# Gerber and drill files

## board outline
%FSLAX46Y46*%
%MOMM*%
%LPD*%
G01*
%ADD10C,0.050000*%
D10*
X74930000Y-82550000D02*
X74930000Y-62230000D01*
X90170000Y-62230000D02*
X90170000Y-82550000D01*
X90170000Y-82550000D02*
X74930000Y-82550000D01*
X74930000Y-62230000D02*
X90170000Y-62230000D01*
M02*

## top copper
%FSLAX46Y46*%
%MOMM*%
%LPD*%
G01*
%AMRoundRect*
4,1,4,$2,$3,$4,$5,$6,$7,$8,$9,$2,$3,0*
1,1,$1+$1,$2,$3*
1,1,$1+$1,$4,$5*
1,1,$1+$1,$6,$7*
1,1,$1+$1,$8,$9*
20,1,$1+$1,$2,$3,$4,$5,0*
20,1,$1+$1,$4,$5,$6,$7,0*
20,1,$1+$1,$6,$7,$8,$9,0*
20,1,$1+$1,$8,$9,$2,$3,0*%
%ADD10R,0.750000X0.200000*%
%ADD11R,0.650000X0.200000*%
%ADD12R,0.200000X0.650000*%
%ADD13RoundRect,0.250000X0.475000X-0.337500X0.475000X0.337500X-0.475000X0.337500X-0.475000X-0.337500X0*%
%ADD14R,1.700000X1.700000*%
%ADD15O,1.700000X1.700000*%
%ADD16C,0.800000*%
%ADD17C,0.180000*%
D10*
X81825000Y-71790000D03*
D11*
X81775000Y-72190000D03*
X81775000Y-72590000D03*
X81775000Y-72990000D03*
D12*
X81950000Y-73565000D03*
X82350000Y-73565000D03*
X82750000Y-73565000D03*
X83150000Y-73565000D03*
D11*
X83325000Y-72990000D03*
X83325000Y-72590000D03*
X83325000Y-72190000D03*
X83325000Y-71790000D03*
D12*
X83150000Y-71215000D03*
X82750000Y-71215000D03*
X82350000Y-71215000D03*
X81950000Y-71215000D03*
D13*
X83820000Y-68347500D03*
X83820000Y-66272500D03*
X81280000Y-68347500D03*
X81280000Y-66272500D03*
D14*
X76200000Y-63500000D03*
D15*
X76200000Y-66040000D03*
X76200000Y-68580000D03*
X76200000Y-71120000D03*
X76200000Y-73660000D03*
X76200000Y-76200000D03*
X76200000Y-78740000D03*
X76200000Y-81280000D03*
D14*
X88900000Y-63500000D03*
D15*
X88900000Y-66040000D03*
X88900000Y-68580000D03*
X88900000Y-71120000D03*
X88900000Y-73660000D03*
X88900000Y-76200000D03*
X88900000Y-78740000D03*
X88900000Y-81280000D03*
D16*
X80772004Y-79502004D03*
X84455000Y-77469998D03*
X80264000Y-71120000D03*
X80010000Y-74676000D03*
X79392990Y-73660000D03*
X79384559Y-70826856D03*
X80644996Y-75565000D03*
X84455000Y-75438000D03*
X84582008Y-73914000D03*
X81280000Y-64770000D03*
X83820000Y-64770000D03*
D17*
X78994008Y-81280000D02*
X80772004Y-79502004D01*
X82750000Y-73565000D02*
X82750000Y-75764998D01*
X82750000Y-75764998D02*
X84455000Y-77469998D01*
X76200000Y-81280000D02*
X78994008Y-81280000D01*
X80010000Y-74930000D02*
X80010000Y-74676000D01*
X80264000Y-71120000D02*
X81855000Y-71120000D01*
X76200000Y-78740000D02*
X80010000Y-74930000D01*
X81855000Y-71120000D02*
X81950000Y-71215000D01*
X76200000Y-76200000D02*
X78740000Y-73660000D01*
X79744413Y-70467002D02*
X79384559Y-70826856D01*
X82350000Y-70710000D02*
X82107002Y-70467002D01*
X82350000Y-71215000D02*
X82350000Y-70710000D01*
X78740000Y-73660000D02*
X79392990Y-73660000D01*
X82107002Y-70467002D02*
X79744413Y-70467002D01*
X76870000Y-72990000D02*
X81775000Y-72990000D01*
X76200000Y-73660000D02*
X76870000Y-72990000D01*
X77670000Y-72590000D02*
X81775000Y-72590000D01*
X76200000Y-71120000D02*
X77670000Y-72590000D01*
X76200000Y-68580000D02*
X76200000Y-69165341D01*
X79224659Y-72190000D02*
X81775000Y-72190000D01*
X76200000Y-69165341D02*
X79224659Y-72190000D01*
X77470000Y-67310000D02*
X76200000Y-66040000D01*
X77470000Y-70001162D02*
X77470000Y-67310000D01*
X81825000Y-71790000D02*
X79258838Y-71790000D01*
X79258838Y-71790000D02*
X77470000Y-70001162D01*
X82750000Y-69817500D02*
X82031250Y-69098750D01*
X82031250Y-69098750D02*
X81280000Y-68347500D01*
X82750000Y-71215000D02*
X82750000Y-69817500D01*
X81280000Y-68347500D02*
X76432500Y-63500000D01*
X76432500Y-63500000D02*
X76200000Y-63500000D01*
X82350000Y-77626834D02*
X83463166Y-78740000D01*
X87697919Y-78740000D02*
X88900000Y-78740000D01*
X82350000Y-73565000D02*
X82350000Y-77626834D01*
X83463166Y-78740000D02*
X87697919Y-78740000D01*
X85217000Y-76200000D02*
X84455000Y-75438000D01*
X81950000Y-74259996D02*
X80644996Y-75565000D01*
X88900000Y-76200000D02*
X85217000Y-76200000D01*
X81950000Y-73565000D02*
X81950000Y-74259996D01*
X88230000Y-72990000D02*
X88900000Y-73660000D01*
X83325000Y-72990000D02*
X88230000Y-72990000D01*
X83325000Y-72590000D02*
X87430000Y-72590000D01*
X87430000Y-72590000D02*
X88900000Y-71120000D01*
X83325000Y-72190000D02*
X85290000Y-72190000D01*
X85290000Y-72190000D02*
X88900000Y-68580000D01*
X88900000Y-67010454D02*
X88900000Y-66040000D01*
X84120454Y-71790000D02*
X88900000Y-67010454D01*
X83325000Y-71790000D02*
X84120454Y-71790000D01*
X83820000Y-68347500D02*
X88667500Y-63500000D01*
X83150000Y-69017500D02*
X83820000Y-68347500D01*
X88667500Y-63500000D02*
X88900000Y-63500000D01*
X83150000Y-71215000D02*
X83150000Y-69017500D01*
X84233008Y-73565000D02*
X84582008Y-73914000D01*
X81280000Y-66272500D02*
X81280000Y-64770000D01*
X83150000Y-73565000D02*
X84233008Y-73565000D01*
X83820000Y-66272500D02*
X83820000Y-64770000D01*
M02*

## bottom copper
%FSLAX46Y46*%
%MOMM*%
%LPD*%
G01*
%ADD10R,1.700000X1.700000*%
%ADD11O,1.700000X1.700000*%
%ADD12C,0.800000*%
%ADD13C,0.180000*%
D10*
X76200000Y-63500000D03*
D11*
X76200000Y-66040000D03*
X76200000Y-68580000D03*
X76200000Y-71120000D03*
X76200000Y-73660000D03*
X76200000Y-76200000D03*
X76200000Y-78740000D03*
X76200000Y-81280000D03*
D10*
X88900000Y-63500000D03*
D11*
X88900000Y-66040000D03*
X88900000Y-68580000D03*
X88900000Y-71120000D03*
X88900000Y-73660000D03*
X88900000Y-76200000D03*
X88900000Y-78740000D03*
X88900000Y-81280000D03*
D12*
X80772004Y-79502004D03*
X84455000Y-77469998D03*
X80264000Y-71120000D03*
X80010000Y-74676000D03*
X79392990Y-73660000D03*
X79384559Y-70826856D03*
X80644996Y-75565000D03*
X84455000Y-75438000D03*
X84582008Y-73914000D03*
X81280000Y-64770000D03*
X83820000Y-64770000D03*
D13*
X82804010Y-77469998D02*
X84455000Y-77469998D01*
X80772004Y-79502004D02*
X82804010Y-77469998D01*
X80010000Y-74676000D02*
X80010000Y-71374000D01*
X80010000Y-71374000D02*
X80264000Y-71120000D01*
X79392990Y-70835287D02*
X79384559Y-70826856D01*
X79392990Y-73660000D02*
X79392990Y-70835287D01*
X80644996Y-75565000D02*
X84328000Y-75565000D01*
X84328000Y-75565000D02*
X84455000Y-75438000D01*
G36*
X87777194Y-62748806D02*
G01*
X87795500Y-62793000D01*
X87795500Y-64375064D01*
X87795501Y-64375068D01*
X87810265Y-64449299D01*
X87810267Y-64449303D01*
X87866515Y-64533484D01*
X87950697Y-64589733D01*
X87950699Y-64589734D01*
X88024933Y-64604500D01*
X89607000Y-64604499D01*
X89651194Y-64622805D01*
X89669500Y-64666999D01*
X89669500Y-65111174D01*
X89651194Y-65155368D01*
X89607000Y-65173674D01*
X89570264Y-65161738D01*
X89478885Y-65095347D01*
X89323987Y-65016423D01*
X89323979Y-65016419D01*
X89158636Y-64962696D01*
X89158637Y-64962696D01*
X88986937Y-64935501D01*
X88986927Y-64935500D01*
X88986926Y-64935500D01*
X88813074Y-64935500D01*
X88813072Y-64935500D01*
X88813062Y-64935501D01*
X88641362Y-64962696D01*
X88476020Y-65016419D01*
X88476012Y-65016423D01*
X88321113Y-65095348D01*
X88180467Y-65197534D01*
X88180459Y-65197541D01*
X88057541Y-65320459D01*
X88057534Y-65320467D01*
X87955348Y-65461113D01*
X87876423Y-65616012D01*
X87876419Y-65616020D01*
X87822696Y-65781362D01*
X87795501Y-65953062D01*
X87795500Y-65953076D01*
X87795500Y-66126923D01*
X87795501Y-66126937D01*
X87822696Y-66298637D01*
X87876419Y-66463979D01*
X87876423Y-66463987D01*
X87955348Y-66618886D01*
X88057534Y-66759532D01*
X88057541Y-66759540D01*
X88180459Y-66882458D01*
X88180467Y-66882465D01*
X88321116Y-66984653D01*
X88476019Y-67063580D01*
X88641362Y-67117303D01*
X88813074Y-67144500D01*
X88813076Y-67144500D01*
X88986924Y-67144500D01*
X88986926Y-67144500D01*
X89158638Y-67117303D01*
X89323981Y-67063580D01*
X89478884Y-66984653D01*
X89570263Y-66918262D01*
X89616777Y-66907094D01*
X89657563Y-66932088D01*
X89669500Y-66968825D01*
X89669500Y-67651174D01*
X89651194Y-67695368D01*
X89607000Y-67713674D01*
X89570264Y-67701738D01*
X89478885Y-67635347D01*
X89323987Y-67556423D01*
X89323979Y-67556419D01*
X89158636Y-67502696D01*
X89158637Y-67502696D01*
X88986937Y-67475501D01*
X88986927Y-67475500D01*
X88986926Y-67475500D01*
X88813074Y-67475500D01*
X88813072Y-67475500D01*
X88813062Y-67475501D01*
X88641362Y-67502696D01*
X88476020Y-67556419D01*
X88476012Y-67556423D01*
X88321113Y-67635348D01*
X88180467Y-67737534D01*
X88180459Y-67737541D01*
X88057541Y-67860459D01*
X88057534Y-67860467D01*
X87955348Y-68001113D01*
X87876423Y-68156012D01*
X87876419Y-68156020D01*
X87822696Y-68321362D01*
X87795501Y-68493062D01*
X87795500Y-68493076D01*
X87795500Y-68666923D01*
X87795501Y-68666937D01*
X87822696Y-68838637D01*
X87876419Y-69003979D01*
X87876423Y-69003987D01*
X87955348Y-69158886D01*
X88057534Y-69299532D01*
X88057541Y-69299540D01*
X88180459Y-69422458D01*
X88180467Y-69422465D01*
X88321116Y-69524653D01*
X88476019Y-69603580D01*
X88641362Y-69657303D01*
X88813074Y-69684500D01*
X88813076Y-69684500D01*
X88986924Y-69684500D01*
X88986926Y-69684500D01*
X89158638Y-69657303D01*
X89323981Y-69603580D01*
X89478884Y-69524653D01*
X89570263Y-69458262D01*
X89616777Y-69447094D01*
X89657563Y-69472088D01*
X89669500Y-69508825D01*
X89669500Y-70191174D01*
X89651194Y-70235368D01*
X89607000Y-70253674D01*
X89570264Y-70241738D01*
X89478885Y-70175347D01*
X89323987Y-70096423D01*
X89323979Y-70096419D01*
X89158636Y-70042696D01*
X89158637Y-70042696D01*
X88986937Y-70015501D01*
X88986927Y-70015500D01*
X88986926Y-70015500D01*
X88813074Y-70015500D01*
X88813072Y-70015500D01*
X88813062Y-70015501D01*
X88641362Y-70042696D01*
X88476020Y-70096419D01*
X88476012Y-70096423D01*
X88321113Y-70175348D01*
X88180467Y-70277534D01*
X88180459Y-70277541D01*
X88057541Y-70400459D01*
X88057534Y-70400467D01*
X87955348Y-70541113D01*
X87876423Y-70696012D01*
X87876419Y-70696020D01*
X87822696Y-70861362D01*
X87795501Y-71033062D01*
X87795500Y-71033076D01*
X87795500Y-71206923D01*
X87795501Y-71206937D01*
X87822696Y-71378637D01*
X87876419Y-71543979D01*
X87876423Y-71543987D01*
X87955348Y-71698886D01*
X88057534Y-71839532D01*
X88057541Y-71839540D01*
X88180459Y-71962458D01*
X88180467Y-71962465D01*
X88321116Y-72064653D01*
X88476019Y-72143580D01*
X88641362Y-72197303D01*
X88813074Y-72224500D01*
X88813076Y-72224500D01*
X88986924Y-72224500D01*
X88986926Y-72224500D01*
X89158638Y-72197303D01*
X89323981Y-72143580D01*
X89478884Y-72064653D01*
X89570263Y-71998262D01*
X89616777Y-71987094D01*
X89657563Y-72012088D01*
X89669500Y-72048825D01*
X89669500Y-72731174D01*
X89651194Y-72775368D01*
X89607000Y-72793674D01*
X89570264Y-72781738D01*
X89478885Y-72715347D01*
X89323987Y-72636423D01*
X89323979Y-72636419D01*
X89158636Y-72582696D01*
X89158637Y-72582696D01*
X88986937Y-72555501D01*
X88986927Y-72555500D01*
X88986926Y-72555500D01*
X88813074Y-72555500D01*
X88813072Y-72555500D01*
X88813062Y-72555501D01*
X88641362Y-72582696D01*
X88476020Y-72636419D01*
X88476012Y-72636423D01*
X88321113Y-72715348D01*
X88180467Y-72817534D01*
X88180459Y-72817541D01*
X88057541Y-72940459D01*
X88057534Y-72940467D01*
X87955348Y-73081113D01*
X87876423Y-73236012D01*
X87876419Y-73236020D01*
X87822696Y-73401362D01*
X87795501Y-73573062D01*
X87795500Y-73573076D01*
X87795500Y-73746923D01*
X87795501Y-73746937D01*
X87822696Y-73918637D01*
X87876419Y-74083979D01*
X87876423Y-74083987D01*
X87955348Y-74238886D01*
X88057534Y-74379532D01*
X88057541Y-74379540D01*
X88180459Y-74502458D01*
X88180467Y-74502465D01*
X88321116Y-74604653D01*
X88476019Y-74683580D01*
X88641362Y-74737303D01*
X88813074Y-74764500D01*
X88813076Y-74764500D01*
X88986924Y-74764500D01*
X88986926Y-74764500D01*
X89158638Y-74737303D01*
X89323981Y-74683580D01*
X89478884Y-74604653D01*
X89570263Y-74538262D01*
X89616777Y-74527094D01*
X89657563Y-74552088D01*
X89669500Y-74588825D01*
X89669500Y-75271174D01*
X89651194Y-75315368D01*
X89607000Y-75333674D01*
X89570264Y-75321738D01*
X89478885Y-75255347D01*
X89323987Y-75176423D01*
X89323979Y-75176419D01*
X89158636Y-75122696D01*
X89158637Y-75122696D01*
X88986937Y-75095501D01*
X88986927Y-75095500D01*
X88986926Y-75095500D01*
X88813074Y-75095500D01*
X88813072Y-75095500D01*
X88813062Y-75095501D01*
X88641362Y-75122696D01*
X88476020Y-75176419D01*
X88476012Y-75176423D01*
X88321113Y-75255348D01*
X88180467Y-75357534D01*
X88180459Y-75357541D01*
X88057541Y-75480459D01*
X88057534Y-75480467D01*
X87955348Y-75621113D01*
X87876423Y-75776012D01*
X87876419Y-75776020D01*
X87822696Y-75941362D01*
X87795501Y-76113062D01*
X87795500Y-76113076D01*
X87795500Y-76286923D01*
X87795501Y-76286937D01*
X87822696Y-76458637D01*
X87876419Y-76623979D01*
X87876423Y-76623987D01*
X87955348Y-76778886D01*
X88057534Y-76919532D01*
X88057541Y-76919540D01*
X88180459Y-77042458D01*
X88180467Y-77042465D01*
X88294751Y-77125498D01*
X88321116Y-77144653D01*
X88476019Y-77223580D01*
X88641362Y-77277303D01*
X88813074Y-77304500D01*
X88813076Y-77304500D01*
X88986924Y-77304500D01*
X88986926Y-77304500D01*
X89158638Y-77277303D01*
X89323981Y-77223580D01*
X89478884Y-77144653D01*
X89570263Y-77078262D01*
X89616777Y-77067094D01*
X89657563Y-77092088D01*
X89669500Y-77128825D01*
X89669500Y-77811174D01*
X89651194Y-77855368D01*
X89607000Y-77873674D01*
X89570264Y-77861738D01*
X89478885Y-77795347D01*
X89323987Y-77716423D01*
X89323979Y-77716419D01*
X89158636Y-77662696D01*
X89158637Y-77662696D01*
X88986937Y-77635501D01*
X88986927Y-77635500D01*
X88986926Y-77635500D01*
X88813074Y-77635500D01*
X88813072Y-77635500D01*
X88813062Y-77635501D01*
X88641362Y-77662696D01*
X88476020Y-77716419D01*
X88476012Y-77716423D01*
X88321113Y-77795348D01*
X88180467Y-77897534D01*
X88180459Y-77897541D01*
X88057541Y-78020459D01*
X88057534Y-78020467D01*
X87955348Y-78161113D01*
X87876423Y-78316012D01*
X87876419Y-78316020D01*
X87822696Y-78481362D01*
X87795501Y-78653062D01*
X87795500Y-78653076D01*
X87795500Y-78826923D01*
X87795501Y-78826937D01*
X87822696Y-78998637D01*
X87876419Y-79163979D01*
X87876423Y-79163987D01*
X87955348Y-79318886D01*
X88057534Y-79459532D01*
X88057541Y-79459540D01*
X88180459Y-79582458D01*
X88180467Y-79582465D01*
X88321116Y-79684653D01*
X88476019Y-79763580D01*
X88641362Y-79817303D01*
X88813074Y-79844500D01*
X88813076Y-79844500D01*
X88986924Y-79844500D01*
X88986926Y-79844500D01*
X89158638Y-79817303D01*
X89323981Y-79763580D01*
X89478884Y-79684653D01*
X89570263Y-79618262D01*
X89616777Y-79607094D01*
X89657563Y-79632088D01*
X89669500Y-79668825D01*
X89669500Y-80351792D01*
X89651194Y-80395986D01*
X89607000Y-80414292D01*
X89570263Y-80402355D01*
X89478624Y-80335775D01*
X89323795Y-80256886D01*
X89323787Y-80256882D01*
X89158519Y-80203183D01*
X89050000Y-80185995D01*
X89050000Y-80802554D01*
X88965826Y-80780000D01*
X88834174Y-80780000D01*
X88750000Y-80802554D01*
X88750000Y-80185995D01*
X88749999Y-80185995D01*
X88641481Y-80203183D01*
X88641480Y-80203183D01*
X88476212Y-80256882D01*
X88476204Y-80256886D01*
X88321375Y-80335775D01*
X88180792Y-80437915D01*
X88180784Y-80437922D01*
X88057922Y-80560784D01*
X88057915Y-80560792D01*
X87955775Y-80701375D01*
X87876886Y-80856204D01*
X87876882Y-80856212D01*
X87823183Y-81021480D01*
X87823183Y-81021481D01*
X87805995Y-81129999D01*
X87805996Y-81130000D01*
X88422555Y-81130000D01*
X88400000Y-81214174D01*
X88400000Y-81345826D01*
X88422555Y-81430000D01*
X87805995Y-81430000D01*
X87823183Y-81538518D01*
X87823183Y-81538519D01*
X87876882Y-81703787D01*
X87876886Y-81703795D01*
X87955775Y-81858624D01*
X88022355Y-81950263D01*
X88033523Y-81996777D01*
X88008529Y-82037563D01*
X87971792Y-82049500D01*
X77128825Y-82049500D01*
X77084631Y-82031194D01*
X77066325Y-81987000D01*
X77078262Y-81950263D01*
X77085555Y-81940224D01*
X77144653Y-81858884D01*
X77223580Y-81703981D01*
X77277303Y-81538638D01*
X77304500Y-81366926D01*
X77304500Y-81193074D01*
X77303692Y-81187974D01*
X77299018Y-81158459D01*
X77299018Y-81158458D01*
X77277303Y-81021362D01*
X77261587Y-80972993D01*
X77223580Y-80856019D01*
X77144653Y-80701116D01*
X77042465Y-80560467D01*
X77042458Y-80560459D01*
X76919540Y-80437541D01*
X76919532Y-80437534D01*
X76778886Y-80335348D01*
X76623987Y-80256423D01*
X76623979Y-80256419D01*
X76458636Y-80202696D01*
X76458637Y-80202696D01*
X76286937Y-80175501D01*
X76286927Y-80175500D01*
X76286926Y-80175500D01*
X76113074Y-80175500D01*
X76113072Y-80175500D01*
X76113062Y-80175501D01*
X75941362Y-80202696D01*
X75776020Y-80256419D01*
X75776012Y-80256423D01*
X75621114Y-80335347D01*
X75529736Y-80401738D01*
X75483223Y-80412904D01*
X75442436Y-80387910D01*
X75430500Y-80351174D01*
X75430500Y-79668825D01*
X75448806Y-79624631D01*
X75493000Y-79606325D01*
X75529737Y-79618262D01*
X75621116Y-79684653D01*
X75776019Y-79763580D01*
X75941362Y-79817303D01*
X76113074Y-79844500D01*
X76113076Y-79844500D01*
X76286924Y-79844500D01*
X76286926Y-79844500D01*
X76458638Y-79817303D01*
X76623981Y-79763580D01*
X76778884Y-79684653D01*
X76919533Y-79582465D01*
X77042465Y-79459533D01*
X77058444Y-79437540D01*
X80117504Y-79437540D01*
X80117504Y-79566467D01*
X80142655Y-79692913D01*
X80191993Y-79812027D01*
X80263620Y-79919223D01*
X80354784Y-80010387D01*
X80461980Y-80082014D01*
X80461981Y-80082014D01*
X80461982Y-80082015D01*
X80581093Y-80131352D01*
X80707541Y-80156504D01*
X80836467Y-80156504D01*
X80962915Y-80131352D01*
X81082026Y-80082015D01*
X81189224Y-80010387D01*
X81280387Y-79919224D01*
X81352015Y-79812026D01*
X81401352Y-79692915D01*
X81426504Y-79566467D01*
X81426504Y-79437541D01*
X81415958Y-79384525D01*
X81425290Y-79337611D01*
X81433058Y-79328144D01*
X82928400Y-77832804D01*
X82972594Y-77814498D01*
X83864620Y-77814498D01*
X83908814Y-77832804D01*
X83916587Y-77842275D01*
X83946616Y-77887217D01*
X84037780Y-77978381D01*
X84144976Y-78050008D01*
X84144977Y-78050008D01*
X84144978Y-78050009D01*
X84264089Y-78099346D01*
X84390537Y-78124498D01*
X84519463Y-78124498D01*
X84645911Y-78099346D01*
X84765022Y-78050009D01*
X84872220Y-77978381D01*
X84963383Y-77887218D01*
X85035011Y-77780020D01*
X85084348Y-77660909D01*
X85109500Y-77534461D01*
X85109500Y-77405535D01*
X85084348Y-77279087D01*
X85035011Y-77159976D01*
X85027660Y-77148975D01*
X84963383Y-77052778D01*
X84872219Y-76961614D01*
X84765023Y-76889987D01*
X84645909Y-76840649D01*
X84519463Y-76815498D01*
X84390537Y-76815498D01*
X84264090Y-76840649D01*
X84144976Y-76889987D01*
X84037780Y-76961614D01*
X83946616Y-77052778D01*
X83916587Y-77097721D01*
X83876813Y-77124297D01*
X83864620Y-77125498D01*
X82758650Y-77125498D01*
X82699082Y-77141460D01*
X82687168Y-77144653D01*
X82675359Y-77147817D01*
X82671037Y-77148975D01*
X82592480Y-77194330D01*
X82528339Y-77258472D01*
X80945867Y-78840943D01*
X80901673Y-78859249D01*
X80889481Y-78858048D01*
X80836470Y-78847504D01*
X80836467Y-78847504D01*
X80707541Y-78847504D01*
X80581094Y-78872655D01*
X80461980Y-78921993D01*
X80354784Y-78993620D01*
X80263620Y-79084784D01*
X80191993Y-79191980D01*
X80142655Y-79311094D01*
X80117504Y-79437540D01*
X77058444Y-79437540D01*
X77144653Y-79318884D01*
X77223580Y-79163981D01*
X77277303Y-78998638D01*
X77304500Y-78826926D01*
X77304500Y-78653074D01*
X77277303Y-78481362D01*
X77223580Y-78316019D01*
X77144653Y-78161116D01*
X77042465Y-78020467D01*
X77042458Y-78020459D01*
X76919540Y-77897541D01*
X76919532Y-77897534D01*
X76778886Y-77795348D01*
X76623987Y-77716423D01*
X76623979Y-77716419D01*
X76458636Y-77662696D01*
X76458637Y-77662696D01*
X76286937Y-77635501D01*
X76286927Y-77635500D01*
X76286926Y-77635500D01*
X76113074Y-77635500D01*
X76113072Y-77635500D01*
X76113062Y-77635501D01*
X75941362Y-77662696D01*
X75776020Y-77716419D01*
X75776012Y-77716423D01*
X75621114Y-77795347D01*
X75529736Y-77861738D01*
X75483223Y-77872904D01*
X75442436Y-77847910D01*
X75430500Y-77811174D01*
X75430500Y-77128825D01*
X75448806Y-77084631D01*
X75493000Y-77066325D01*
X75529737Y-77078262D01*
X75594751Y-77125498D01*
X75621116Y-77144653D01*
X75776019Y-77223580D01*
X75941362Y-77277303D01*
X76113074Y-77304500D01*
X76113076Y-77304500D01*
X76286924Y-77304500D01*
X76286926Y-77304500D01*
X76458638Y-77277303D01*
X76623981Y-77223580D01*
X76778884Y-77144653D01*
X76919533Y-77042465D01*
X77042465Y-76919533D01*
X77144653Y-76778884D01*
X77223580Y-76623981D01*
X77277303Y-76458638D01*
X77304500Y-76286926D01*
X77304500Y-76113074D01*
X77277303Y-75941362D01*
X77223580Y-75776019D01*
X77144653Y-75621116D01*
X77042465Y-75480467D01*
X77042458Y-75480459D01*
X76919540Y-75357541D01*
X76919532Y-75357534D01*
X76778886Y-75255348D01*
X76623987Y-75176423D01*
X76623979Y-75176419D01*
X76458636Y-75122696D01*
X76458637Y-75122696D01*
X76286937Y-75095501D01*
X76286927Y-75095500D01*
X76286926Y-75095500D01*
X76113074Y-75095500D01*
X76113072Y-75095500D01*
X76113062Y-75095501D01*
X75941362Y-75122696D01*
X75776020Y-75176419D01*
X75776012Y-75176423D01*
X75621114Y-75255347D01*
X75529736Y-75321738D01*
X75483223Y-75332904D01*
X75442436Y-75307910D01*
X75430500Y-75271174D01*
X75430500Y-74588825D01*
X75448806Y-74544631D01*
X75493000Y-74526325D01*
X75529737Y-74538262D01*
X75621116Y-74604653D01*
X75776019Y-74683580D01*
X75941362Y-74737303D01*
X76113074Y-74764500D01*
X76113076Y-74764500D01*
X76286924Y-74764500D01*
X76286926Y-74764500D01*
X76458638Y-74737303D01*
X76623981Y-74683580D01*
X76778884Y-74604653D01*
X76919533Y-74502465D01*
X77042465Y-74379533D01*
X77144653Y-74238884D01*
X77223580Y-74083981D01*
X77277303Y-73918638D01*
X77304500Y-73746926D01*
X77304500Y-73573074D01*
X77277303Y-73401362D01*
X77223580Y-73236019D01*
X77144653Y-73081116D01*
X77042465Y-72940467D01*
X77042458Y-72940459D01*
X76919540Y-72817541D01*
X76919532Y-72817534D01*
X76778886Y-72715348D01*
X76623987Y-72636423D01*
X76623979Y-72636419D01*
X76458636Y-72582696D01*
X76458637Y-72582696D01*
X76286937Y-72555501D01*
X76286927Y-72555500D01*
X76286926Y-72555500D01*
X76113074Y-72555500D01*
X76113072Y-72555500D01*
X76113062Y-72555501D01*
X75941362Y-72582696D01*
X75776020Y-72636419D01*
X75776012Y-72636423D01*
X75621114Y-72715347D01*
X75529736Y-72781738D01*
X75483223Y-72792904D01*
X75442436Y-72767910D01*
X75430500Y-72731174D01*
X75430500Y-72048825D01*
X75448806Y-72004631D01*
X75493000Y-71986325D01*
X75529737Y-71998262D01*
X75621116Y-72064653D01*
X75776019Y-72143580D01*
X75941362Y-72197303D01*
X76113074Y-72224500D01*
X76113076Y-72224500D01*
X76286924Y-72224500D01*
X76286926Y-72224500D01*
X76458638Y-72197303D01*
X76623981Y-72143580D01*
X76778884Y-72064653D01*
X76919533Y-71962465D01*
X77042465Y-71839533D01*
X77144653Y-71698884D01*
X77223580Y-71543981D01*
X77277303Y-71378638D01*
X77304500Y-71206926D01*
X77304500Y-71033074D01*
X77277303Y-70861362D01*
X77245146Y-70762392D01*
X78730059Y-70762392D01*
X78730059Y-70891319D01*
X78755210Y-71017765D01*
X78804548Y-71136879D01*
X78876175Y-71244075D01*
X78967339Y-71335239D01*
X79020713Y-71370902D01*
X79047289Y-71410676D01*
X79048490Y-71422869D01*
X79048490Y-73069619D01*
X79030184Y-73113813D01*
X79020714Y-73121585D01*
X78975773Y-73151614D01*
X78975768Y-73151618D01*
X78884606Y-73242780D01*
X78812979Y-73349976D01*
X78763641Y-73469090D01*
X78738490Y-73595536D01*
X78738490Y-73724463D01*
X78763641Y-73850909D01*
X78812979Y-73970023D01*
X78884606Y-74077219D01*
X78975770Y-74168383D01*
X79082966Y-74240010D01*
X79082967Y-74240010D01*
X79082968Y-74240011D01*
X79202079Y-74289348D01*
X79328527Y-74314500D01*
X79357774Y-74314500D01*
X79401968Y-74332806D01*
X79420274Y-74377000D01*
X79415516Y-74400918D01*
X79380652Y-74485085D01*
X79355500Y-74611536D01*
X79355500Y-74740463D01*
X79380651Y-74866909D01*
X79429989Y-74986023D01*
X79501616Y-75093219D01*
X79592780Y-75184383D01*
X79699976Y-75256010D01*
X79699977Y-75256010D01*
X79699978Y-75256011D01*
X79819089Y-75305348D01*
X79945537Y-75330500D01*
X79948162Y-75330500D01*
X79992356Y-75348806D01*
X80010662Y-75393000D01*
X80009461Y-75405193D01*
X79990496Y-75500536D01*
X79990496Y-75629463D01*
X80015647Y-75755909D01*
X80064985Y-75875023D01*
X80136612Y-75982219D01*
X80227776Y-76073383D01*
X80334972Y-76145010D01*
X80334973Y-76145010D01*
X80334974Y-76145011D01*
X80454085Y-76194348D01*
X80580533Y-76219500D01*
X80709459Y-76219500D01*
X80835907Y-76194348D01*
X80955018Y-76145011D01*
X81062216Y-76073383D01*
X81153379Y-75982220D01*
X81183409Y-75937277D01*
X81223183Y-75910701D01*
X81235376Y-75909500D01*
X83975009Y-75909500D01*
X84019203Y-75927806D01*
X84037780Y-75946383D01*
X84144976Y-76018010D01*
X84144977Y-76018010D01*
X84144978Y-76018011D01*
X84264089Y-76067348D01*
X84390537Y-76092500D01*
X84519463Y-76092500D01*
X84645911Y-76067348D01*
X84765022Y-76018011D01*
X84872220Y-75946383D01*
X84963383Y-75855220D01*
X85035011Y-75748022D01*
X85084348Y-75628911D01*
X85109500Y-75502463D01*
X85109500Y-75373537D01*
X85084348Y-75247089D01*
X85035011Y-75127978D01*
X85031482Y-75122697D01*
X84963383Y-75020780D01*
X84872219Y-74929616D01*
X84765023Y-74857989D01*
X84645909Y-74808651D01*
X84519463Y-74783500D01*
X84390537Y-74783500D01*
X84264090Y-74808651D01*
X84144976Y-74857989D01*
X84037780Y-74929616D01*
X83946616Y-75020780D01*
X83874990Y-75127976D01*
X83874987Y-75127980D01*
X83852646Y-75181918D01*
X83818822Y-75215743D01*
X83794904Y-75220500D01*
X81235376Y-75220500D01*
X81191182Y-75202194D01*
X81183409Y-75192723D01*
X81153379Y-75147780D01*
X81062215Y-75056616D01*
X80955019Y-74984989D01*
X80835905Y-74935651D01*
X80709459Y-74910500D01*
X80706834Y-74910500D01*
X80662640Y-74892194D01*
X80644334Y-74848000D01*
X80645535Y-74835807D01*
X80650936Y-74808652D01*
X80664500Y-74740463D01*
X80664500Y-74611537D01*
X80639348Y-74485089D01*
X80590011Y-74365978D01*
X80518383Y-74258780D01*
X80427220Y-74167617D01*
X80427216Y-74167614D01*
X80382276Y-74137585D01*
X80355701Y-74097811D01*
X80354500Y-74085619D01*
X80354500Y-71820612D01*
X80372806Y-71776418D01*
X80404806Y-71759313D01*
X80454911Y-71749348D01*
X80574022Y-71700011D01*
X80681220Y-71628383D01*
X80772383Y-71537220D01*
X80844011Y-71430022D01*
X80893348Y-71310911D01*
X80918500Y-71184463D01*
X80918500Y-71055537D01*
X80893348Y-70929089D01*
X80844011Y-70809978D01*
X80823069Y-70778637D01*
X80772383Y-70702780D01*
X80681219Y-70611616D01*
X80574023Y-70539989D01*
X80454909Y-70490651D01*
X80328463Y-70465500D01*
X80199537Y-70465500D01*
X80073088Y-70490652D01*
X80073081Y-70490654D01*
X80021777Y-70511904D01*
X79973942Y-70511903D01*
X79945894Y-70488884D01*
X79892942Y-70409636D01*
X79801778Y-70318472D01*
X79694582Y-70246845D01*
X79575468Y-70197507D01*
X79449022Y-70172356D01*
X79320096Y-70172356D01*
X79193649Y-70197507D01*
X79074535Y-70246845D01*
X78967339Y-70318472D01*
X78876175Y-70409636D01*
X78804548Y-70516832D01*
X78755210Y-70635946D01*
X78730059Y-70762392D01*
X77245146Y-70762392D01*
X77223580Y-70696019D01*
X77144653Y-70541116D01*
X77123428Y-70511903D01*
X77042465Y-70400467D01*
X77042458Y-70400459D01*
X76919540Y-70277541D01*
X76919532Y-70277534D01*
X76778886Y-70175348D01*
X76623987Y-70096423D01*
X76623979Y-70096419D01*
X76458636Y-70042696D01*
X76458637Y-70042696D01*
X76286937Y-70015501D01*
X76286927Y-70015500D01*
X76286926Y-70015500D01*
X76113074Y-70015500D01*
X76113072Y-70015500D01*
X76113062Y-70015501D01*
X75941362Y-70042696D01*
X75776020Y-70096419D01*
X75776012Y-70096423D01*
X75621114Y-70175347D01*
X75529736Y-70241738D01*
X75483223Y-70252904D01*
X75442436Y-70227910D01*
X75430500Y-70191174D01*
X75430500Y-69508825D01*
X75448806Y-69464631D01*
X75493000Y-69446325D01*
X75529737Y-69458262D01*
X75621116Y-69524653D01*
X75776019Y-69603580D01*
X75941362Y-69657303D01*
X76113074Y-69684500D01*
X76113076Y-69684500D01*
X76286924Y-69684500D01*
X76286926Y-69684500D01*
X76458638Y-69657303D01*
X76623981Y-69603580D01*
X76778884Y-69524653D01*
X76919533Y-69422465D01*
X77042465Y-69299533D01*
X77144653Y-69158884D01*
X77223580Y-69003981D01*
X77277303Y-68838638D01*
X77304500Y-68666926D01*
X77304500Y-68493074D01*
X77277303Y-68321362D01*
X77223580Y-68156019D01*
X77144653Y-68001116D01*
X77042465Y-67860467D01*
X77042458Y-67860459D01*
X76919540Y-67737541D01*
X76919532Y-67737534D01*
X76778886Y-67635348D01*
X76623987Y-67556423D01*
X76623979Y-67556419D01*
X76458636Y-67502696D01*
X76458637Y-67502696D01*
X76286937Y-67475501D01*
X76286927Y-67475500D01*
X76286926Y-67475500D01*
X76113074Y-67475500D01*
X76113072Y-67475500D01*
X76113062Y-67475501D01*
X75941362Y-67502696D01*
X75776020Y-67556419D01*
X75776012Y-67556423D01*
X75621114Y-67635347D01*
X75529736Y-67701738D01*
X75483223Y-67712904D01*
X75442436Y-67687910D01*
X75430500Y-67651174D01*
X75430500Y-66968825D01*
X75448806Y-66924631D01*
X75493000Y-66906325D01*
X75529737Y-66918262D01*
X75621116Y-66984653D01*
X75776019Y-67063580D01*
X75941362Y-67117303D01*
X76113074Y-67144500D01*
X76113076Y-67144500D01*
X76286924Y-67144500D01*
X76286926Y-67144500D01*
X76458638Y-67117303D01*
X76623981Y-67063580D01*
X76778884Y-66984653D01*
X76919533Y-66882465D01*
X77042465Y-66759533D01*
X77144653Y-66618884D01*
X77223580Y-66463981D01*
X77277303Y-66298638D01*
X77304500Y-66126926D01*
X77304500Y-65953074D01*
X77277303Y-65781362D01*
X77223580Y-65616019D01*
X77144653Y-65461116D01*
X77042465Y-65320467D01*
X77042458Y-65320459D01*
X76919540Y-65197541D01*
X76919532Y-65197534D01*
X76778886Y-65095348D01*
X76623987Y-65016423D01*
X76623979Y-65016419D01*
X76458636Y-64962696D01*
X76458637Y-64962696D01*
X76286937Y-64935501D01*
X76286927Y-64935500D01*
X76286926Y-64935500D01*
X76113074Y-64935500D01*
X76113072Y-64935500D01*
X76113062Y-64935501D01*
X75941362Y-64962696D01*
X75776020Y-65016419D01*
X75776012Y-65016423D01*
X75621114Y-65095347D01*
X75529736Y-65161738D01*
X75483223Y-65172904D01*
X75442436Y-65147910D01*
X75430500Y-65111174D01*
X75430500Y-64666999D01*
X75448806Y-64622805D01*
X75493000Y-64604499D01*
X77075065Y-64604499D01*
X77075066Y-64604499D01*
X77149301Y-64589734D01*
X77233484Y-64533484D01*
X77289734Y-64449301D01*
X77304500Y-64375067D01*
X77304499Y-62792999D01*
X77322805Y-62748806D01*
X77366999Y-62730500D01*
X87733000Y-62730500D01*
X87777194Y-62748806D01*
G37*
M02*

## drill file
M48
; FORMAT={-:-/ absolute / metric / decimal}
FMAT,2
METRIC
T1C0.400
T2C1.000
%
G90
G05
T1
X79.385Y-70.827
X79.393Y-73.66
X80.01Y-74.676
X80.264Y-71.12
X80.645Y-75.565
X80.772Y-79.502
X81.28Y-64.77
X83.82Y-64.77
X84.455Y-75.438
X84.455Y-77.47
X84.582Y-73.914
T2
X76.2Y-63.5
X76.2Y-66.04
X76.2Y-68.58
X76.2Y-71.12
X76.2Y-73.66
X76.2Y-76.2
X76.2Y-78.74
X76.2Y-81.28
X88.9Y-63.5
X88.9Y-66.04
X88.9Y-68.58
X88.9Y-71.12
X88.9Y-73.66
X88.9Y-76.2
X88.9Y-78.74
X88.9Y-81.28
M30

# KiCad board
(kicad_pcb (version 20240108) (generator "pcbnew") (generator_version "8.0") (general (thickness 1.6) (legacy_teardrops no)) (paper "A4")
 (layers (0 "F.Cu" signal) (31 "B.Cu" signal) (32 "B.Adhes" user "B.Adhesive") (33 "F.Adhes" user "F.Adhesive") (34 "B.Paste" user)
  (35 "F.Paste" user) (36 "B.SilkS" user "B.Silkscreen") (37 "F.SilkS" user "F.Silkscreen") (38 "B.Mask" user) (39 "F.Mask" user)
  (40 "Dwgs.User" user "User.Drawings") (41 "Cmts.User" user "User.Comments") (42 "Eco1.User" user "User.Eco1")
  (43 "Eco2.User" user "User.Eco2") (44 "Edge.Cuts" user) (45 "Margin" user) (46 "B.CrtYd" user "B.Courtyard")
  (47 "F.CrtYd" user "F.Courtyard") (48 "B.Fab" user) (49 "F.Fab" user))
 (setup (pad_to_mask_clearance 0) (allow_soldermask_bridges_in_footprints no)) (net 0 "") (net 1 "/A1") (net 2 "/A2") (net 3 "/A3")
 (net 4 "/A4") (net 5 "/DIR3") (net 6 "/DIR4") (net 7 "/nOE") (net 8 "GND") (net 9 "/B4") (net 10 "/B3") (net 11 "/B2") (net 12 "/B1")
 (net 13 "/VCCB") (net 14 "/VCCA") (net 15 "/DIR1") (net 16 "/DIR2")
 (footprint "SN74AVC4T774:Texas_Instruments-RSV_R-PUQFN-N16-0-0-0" (layer "F.Cu") (at 82.55 72.39 -90)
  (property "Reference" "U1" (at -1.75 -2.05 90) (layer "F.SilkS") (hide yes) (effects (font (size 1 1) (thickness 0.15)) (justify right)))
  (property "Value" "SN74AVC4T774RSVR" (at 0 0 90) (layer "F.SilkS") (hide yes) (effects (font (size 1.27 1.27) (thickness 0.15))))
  (pad "1" smd rect (at -0.6 0.725 270) (size 0.2 0.75) (layers "F.Cu" "F.Paste" "F.Mask") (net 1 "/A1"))
  (pad "2" smd rect (at -0.2 0.775 270) (size 0.2 0.65) (layers "F.Cu" "F.Paste" "F.Mask") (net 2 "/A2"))
  (pad "3" smd rect (at 0.2 0.775 270) (size 0.2 0.65) (layers "F.Cu" "F.Paste" "F.Mask") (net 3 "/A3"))
  (pad "4" smd rect (at 0.6 0.775 270) (size 0.2 0.65) (layers "F.Cu" "F.Paste" "F.Mask") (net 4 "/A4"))
  (pad "5" smd rect (at 1.175 0.6 270) (size 0.65 0.2) (layers "F.Cu" "F.Paste" "F.Mask") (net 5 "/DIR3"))
  (pad "6" smd rect (at 1.175 0.2 270) (size 0.65 0.2) (layers "F.Cu" "F.Paste" "F.Mask") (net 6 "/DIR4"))
  (pad "7" smd rect (at 1.175 -0.2 270) (size 0.65 0.2) (layers "F.Cu" "F.Paste" "F.Mask") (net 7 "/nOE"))
  (pad "8" smd rect (at 1.175 -0.6 270) (size 0.65 0.2) (layers "F.Cu" "F.Paste" "F.Mask") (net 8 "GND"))
  (pad "9" smd rect (at 0.6 -0.775 270) (size 0.2 0.65) (layers "F.Cu" "F.Paste" "F.Mask") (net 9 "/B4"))
  (pad "10" smd rect (at 0.2 -0.775 270) (size 0.2 0.65) (layers "F.Cu" "F.Paste" "F.Mask") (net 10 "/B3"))
  (pad "11" smd rect (at -0.2 -0.775 270) (size 0.2 0.65) (layers "F.Cu" "F.Paste" "F.Mask") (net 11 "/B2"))
  (pad "12" smd rect (at -0.6 -0.775 270) (size 0.2 0.65) (layers "F.Cu" "F.Paste" "F.Mask") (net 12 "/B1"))
  (pad "13" smd rect (at -1.175 -0.6 270) (size 0.65 0.2) (layers "F.Cu" "F.Paste" "F.Mask") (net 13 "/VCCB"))
  (pad "14" smd rect (at -1.175 -0.2 270) (size 0.65 0.2) (layers "F.Cu" "F.Paste" "F.Mask") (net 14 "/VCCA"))
  (pad "15" smd rect (at -1.175 0.2 270) (size 0.65 0.2) (layers "F.Cu" "F.Paste" "F.Mask") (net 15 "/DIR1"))
  (pad "16" smd rect (at -1.175 0.6 270) (size 0.65 0.2) (layers "F.Cu" "F.Paste" "F.Mask") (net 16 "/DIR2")))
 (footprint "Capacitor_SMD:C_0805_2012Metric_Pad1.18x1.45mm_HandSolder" (layer "F.Cu") (at 83.82 67.31 90)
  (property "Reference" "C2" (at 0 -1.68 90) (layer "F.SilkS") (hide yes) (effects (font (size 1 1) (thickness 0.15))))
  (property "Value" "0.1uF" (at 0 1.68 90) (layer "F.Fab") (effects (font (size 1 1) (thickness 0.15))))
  (pad "1" smd roundrect (at -1.0375 0 90) (size 1.175 1.45) (layers "F.Cu" "F.Paste" "F.Mask") (roundrect_rratio 0.212766) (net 13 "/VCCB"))
  (pad "2" smd roundrect (at 1.0375 0 90) (size 1.175 1.45) (layers "F.Cu" "F.Paste" "F.Mask") (roundrect_rratio 0.212766) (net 8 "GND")))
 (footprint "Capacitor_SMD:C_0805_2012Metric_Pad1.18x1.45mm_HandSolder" (layer "F.Cu") (at 81.28 67.31 90)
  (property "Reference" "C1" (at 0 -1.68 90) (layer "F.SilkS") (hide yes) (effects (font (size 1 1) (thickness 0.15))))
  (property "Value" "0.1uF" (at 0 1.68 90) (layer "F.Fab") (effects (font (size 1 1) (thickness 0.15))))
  (pad "1" smd roundrect (at -1.0375 0 90) (size 1.175 1.45) (layers "F.Cu" "F.Paste" "F.Mask") (roundrect_rratio 0.212766) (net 14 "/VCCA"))
  (pad "2" smd roundrect (at 1.0375 0 90) (size 1.175 1.45) (layers "F.Cu" "F.Paste" "F.Mask") (roundrect_rratio 0.212766) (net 8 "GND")))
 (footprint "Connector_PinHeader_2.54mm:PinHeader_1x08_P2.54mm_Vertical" (layer "B.Cu") (at 76.2 63.5 180)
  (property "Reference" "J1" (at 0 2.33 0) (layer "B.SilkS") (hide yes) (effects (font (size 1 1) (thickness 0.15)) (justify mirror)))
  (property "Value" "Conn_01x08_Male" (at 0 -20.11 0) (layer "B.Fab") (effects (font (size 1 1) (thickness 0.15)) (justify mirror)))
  (pad "1" thru_hole rect (at 0 0 180) (size 1.7 1.7) (drill 1) (layers "*.Cu" "*.Mask") (remove_unused_layers no) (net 14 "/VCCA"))
  (pad "2" thru_hole oval (at 0 -2.54 180) (size 1.7 1.7) (drill 1) (layers "*.Cu" "*.Mask") (remove_unused_layers no) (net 1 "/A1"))
  (pad "3" thru_hole oval (at 0 -5.08 180) (size 1.7 1.7) (drill 1) (layers "*.Cu" "*.Mask") (remove_unused_layers no) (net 2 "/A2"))
  (pad "4" thru_hole oval (at 0 -7.62 180) (size 1.7 1.7) (drill 1) (layers "*.Cu" "*.Mask") (remove_unused_layers no) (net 3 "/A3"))
  (pad "5" thru_hole oval (at 0 -10.16 180) (size 1.7 1.7) (drill 1) (layers "*.Cu" "*.Mask") (remove_unused_layers no) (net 4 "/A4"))
  (pad "6" thru_hole oval (at 0 -12.7 180) (size 1.7 1.7) (drill 1) (layers "*.Cu" "*.Mask") (remove_unused_layers no) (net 15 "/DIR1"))
  (pad "7" thru_hole oval (at 0 -15.24 180) (size 1.7 1.7) (drill 1) (layers "*.Cu" "*.Mask") (remove_unused_layers no) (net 16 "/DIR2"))
  (pad "8" thru_hole oval (at 0 -17.78 180) (size 1.7 1.7) (drill 1) (layers "*.Cu" "*.Mask") (remove_unused_layers no) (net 7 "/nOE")))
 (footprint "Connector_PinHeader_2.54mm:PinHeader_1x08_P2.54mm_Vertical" (layer "B.Cu") (at 88.9 63.5 180)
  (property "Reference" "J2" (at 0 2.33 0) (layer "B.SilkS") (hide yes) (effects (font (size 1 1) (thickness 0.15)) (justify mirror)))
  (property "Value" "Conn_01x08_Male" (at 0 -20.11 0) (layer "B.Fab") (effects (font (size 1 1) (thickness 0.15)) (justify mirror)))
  (pad "1" thru_hole rect (at 0 0 180) (size 1.7 1.7) (drill 1) (layers "*.Cu" "*.Mask") (remove_unused_layers no) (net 13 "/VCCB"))
  (pad "2" thru_hole oval (at 0 -2.54 180) (size 1.7 1.7) (drill 1) (layers "*.Cu" "*.Mask") (remove_unused_layers no) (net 12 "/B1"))
  (pad "3" thru_hole oval (at 0 -5.08 180) (size 1.7 1.7) (drill 1) (layers "*.Cu" "*.Mask") (remove_unused_layers no) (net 11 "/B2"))
  (pad "4" thru_hole oval (at 0 -7.62 180) (size 1.7 1.7) (drill 1) (layers "*.Cu" "*.Mask") (remove_unused_layers no) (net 10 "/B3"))
  (pad "5" thru_hole oval (at 0 -10.16 180) (size 1.7 1.7) (drill 1) (layers "*.Cu" "*.Mask") (remove_unused_layers no) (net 9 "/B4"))
  (pad "6" thru_hole oval (at 0 -12.7 180) (size 1.7 1.7) (drill 1) (layers "*.Cu" "*.Mask") (remove_unused_layers no) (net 5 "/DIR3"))
  (pad "7" thru_hole oval (at 0 -15.24 180) (size 1.7 1.7) (drill 1) (layers "*.Cu" "*.Mask") (remove_unused_layers no) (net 6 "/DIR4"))
  (pad "8" thru_hole oval (at 0 -17.78 180) (size 1.7 1.7) (drill 1) (layers "*.Cu" "*.Mask") (remove_unused_layers no) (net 8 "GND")))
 (gr_line (start 74.93 82.55) (end 74.93 62.23) (stroke (width 0.05) (type solid)) (layer "Edge.Cuts"))
 (gr_line (start 90.17 62.23) (end 90.17 82.55) (stroke (width 0.05) (type solid)) (layer "Edge.Cuts"))
 (gr_line (start 90.17 82.55) (end 74.93 82.55) (stroke (width 0.05) (type solid)) (layer "Edge.Cuts"))
 (gr_line (start 74.93 62.23) (end 90.17 62.23) (stroke (width 0.05) (type solid)) (layer "Edge.Cuts"))
 (segment (start 78.994008 81.28) (end 80.772004 79.502004) (width 0.18) (layer "F.Cu") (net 7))
 (segment (start 82.75 73.565) (end 82.75 75.764998) (width 0.18) (layer "F.Cu") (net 7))
 (segment (start 82.75 75.764998) (end 84.455 77.469998) (width 0.18) (layer "F.Cu") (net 7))
 (segment (start 76.2 81.28) (end 78.994008 81.28) (width 0.18) (layer "F.Cu") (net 7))
 (via (at 80.772004 79.502004) (size 0.8) (drill 0.4) (layers "F.Cu" "B.Cu") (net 7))
 (via (at 84.455 77.469998) (size 0.8) (drill 0.4) (layers "F.Cu" "B.Cu") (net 7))
 (segment (start 82.80401 77.469998) (end 84.455 77.469998) (width 0.18) (layer "B.Cu") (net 7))
 (segment (start 80.772004 79.502004) (end 82.80401 77.469998) (width 0.18) (layer "B.Cu") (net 7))
 (segment (start 80.01 74.93) (end 80.01 74.676) (width 0.18) (layer "F.Cu") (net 16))
 (segment (start 80.264 71.12) (end 81.855 71.12) (width 0.18) (layer "F.Cu") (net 16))
 (segment (start 76.2 78.74) (end 80.01 74.93) (width 0.18) (layer "F.Cu") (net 16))
 (segment (start 81.855 71.12) (end 81.95 71.215) (width 0.18) (layer "F.Cu") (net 16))
 (via (at 80.264 71.12) (size 0.8) (drill 0.4) (layers "F.Cu" "B.Cu") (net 16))
 (via (at 80.01 74.676) (size 0.8) (drill 0.4) (layers "F.Cu" "B.Cu") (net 16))
 (segment (start 80.01 74.676) (end 80.01 71.374) (width 0.18) (layer "B.Cu") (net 16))
 (segment (start 80.01 71.374) (end 80.264 71.12) (width 0.18) (layer "B.Cu") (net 16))
 (segment (start 76.2 76.2) (end 78.74 73.66) (width 0.18) (layer "F.Cu") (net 15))
 (segment (start 79.744413 70.467002) (end 79.384559 70.826856) (width 0.18) (layer "F.Cu") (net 15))
 (segment (start 82.35 70.71) (end 82.107002 70.467002) (width 0.18) (layer "F.Cu") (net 15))
 (segment (start 82.35 71.215) (end 82.35 70.71) (width 0.18) (layer "F.Cu") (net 15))
 (segment (start 78.74 73.66) (end 79.39299 73.66) (width 0.18) (layer "F.Cu") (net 15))
 (segment (start 82.107002 70.467002) (end 79.744413 70.467002) (width 0.18) (layer "F.Cu") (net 15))
 (via (at 79.39299 73.66) (size 0.8) (drill 0.4) (layers "F.Cu" "B.Cu") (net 15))
 (via (at 79.384559 70.826856) (size 0.8) (drill 0.4) (layers "F.Cu" "B.Cu") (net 15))
 (segment (start 79.39299 70.835287) (end 79.384559 70.826856) (width 0.18) (layer "B.Cu") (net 15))
 (segment (start 79.39299 73.66) (end 79.39299 70.835287) (width 0.18) (layer "B.Cu") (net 15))
 (segment (start 76.87 72.99) (end 81.775 72.99) (width 0.18) (layer "F.Cu") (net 4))
 (segment (start 76.2 73.66) (end 76.87 72.99) (width 0.18) (layer "F.Cu") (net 4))
 (segment (start 77.67 72.59) (end 81.775 72.59) (width 0.18) (layer "F.Cu") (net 3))
 (segment (start 76.2 71.12) (end 77.67 72.59) (width 0.18) (layer "F.Cu") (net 3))
 (segment (start 76.2 68.58) (end 76.2 69.165341) (width 0.18) (layer "F.Cu") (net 2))
 (segment (start 79.224659 72.19) (end 81.775 72.19) (width 0.18) (layer "F.Cu") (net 2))
 (segment (start 76.2 69.165341) (end 79.224659 72.19) (width 0.18) (layer "F.Cu") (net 2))
 (segment (start 77.47 67.31) (end 76.2 66.04) (width 0.18) (layer "F.Cu") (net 1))
 (segment (start 77.47 70.001162) (end 77.47 67.31) (width 0.18) (layer "F.Cu") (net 1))
 (segment (start 81.825 71.79) (end 79.258838 71.79) (width 0.18) (layer "F.Cu") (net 1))
 (segment (start 79.258838 71.79) (end 77.47 70.001162) (width 0.18) (layer "F.Cu") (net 1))
 (segment (start 82.75 69.8175) (end 82.03125 69.09875) (width 0.18) (layer "F.Cu") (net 14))
 (segment (start 82.03125 69.09875) (end 81.28 68.3475) (width 0.18) (layer "F.Cu") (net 14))
 (segment (start 82.75 71.215) (end 82.75 69.8175) (width 0.18) (layer "F.Cu") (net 14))
 (segment (start 81.28 68.3475) (end 76.4325 63.5) (width 0.18) (layer "F.Cu") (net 14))
 (segment (start 76.4325 63.5) (end 76.2 63.5) (width 0.18) (layer "F.Cu") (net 14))
 (segment (start 82.35 77.626834) (end 83.463166 78.74) (width 0.18) (layer "F.Cu") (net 6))
 (segment (start 87.697919 78.74) (end 88.9 78.74) (width 0.18) (layer "F.Cu") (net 6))
 (segment (start 82.35 73.565) (end 82.35 77.626834) (width 0.18) (layer "F.Cu") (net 6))
 (segment (start 83.463166 78.74) (end 87.697919 78.74) (width 0.18) (layer "F.Cu") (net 6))
 (segment (start 85.217 76.2) (end 84.455 75.438) (width 0.18) (layer "F.Cu") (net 5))
 (segment (start 81.95 74.259996) (end 80.644996 75.565) (width 0.18) (layer "F.Cu") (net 5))
 (segment (start 88.9 76.2) (end 85.217 76.2) (width 0.18) (layer "F.Cu") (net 5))
 (segment (start 81.95 73.565) (end 81.95 74.259996) (width 0.18) (layer "F.Cu") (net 5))
 (via (at 80.644996 75.565) (size 0.8) (drill 0.4) (layers "F.Cu" "B.Cu") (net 5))
 (via (at 84.455 75.438) (size 0.8) (drill 0.4) (layers "F.Cu" "B.Cu") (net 5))
 (segment (start 80.644996 75.565) (end 84.328 75.565) (width 0.18) (layer "B.Cu") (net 5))
 (segment (start 84.328 75.565) (end 84.455 75.438) (width 0.18) (layer "B.Cu") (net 5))
 (segment (start 88.23 72.99) (end 88.9 73.66) (width 0.18) (layer "F.Cu") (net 9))
 (segment (start 83.325 72.99) (end 88.23 72.99) (width 0.18) (layer "F.Cu") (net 9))
 (segment (start 83.325 72.59) (end 87.43 72.59) (width 0.18) (layer "F.Cu") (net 10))
 (segment (start 87.43 72.59) (end 88.9 71.12) (width 0.18) (layer "F.Cu") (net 10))
 (segment (start 83.325 72.19) (end 85.29 72.19) (width 0.18) (layer "F.Cu") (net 11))
 (segment (start 85.29 72.19) (end 88.9 68.58) (width 0.18) (layer "F.Cu") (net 11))
 (segment (start 88.9 67.010454) (end 88.9 66.04) (width 0.18) (layer "F.Cu") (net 12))
 (segment (start 84.120454 71.79) (end 88.9 67.010454) (width 0.18) (layer "F.Cu") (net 12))
 (segment (start 83.325 71.79) (end 84.120454 71.79) (width 0.18) (layer "F.Cu") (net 12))
 (segment (start 83.82 68.3475) (end 88.6675 63.5) (width 0.18) (layer "F.Cu") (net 13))
 (segment (start 83.15 69.0175) (end 83.82 68.3475) (width 0.18) (layer "F.Cu") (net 13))
 (segment (start 88.6675 63.5) (end 88.9 63.5) (width 0.18) (layer "F.Cu") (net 13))
 (segment (start 83.15 71.215) (end 83.15 69.0175) (width 0.18) (layer "F.Cu") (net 13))
 (segment (start 84.233008 73.565) (end 84.582008 73.914) (width 0.18) (layer "F.Cu") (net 8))
 (segment (start 81.28 66.2725) (end 81.28 64.77) (width 0.18) (layer "F.Cu") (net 8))
 (segment (start 83.15 73.565) (end 84.233008 73.565) (width 0.18) (layer "F.Cu") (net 8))
 (segment (start 83.82 66.2725) (end 83.82 64.77) (width 0.18) (layer "F.Cu") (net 8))
 (via (at 84.582008 73.914) (size 0.8) (drill 0.4) (layers "F.Cu" "B.Cu") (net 8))
 (via (at 81.28 64.77) (size 0.8) (drill 0.4) (layers "F.Cu" "B.Cu") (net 8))
 (via (at 83.82 64.77) (size 0.8) (drill 0.4) (layers "F.Cu" "B.Cu") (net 8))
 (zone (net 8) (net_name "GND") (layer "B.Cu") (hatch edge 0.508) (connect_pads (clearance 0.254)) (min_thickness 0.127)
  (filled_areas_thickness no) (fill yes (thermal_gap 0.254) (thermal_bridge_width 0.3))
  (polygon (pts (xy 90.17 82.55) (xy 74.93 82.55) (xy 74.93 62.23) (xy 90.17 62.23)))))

